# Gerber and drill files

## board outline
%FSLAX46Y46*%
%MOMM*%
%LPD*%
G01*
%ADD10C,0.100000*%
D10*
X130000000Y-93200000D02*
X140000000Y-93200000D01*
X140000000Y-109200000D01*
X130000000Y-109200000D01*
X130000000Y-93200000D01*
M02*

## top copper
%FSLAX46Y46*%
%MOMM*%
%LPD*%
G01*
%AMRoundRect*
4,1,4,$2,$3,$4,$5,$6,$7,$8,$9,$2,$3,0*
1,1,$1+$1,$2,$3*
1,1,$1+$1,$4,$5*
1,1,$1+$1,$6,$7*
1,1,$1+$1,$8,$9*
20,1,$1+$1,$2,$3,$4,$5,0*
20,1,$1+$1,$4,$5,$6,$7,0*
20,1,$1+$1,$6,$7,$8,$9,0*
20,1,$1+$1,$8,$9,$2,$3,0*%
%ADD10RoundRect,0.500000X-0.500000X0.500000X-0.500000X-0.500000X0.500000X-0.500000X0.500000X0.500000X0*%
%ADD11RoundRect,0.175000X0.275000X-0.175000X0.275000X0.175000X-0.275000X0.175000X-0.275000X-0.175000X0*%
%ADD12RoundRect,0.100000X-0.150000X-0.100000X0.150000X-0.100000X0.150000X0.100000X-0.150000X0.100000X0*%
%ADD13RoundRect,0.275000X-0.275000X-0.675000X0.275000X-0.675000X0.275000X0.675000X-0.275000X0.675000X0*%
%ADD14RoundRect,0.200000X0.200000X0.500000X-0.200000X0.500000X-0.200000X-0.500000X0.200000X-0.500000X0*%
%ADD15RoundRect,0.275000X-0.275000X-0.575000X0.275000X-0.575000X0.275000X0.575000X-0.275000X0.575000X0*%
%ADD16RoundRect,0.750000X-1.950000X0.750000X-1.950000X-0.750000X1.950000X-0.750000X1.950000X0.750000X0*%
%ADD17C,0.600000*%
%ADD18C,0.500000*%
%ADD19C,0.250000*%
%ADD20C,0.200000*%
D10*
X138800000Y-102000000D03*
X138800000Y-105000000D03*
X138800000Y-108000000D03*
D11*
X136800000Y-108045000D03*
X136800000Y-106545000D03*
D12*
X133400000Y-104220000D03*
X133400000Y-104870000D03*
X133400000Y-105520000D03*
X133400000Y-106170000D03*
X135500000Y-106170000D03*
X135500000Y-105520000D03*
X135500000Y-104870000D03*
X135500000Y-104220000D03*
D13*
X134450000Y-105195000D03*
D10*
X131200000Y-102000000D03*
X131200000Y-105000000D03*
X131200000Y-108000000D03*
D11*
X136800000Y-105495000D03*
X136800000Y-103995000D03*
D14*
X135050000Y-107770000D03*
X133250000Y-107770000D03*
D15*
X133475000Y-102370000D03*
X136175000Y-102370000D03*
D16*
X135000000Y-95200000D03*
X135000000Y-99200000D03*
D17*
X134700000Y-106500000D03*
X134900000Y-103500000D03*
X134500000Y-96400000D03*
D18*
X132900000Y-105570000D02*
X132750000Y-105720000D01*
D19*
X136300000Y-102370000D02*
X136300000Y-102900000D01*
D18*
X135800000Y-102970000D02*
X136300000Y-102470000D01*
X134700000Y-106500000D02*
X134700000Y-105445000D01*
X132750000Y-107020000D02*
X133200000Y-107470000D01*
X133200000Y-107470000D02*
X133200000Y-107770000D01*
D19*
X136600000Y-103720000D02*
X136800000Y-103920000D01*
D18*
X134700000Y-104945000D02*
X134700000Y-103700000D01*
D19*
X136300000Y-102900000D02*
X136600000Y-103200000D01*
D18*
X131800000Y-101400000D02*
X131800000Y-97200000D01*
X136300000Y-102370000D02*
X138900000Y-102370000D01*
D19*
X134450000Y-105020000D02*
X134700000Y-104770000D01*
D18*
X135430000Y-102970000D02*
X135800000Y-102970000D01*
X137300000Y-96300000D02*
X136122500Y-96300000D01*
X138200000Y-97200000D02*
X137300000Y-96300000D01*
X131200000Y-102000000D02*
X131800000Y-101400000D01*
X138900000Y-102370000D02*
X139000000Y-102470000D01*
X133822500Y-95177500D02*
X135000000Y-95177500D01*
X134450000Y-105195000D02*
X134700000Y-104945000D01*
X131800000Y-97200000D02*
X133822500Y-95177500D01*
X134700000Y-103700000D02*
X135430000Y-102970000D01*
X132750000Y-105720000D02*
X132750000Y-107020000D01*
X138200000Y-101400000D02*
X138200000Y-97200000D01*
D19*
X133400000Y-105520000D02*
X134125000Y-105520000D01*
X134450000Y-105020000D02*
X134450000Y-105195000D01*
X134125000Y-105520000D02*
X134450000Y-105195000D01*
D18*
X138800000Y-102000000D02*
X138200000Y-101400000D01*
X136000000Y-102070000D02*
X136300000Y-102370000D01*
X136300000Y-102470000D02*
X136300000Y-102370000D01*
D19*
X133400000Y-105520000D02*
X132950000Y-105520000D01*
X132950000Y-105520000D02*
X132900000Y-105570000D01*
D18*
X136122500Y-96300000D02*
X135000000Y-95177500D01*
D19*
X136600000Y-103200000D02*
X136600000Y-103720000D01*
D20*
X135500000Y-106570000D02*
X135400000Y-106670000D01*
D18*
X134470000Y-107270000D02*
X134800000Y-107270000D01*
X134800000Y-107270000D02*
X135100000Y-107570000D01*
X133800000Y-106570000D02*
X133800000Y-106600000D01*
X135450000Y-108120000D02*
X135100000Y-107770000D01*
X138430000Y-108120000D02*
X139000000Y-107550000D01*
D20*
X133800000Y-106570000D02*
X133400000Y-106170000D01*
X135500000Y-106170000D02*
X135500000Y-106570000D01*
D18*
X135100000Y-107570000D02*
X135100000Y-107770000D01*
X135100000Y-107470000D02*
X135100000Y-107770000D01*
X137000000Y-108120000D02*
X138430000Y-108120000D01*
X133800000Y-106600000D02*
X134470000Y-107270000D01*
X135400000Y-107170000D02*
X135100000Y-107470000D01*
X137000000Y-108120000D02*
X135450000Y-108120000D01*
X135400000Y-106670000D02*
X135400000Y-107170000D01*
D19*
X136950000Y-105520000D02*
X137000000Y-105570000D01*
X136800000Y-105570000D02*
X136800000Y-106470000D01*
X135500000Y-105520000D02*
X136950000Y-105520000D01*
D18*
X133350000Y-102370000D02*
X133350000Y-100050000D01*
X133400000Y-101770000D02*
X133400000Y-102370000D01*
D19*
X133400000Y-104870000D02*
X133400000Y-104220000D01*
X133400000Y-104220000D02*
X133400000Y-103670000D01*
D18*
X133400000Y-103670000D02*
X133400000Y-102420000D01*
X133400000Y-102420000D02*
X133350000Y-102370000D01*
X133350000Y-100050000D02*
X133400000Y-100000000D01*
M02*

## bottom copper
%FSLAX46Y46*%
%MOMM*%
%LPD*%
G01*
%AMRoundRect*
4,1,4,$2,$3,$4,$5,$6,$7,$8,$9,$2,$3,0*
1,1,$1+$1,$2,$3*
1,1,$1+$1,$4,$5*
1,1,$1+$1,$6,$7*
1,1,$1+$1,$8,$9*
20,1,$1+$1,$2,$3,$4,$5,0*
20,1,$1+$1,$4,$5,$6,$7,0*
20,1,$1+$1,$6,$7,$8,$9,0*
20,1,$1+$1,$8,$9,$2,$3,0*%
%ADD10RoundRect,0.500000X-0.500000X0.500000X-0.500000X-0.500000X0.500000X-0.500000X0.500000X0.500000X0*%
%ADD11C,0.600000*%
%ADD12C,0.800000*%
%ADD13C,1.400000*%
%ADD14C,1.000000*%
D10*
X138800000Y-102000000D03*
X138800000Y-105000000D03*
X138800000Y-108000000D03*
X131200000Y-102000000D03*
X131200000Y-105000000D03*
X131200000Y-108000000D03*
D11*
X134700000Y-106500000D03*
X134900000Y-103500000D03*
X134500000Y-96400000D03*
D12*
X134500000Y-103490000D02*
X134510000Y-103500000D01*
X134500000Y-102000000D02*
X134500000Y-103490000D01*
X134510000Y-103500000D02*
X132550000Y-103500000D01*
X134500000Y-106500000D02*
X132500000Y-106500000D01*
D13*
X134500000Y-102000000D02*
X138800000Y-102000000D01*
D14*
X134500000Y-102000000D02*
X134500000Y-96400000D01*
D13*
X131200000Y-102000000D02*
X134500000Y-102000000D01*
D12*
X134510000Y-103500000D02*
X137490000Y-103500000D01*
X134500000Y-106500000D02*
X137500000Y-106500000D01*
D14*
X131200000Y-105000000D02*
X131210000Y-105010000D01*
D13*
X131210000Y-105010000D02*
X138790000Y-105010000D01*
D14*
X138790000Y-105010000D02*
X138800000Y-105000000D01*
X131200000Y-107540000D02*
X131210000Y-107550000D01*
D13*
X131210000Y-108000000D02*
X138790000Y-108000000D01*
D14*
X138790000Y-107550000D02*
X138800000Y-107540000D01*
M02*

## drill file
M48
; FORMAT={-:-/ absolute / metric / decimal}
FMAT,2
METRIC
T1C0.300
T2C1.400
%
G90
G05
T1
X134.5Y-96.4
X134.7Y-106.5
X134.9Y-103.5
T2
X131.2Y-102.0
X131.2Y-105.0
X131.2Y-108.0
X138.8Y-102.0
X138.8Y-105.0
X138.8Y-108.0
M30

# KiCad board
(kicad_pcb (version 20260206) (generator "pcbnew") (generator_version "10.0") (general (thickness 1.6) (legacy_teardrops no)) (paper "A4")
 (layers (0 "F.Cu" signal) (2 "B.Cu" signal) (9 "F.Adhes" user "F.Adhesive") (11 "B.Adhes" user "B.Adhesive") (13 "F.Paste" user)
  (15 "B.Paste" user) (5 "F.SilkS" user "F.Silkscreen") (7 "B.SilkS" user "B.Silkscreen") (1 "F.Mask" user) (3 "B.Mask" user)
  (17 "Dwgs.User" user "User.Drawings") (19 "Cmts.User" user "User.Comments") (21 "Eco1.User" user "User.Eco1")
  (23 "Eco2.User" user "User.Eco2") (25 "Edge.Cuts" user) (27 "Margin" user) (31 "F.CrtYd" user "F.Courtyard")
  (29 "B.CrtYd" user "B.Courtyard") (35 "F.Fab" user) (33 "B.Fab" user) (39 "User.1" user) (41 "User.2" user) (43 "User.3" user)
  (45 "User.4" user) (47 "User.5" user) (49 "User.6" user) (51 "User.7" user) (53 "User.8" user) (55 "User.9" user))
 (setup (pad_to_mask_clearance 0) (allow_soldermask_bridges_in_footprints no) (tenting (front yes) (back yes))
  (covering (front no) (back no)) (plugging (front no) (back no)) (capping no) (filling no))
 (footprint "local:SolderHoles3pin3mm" (layer "F.Cu") (at 138.8 105 -90)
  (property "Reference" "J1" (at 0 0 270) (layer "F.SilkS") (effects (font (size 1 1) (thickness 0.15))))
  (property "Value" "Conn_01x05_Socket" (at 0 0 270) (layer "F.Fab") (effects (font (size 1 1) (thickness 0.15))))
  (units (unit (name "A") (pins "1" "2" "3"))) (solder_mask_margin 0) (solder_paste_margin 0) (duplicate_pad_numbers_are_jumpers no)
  (pad "1" thru_hole roundrect (at -3 0 270) (size 2 2) (drill 1.4) (layers "*.Cu" "*.Mask") (remove_unused_layers yes)
   (keep_end_layers yes) (zone_layer_connections) (roundrect_rratio 0.25) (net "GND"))
  (pad "2" thru_hole roundrect (at 0 0 270) (size 2 2) (drill 1.4) (layers "*.Cu" "*.Mask") (remove_unused_layers yes) (keep_end_layers yes)
   (zone_layer_connections) (roundrect_rratio 0.25) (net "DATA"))
  (pad "3" thru_hole roundrect (at 3 0 270) (size 2 2) (drill 1.4) (layers "*.Cu" "*.Mask") (remove_unused_layers yes) (keep_end_layers yes)
   (zone_layer_connections) (roundrect_rratio 0.25) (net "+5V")))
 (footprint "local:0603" (layer "F.Cu") (at 136.8 107.295 90)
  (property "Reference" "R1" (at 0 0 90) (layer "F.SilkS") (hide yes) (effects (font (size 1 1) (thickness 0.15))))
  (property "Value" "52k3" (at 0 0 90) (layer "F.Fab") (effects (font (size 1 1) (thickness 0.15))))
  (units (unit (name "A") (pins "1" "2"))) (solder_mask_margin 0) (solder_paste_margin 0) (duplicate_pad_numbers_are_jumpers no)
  (pad "1" smd roundrect (at -0.75 0 90) (size 0.7 0.9) (layers "F.Cu" "F.Mask" "F.Paste") (roundrect_rratio 0.25) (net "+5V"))
  (pad "2" smd roundrect (at 0.75 0 90) (size 0.7 0.9) (layers "F.Cu" "F.Mask" "F.Paste") (roundrect_rratio 0.25) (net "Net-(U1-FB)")))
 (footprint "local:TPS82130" (layer "F.Cu") (at 134.45 105.195)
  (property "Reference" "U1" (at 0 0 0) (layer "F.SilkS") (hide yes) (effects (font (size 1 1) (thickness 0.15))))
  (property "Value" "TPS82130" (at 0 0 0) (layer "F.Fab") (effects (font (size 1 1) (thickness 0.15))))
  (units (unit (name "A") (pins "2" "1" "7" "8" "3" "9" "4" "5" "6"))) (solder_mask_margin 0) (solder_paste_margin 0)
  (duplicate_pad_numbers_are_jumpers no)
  (pad "1" smd roundrect (at -1.05 -0.975) (size 0.5 0.4) (layers "F.Cu" "F.Mask" "F.Paste") (roundrect_rratio 0.25) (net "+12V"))
  (pad "2" smd roundrect (at -1.05 -0.325) (size 0.5 0.4) (layers "F.Cu" "F.Mask" "F.Paste") (roundrect_rratio 0.25) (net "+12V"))
  (pad "3" smd roundrect (at -1.05 0.325) (size 0.5 0.4) (layers "F.Cu" "F.Mask" "F.Paste") (roundrect_rratio 0.25) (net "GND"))
  (pad "4" smd roundrect (at -1.05 0.975) (size 0.5 0.4) (layers "F.Cu" "F.Mask" "F.Paste") (roundrect_rratio 0.25) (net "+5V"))
  (pad "5" smd roundrect (at 1.05 0.975) (size 0.5 0.4) (layers "F.Cu" "F.Mask" "F.Paste") (roundrect_rratio 0.25) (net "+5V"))
  (pad "6" smd roundrect (at 1.05 0.325) (size 0.5 0.4) (layers "F.Cu" "F.Mask" "F.Paste") (roundrect_rratio 0.25) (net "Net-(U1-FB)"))
  (pad "7" smd roundrect (at 1.05 -0.325) (size 0.5 0.4) (layers "F.Cu" "F.Mask" "F.Paste") (roundrect_rratio 0.25)
   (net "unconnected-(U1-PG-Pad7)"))
  (pad "8" smd roundrect (at 1.05 -0.975) (size 0.5 0.4) (layers "F.Cu" "F.Mask" "F.Paste") (roundrect_rratio 0.25)
   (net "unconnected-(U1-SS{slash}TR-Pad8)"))
  (pad "9" smd roundrect (at 0 0) (size 1.1 1.9) (layers "F.Cu" "F.Mask" "F.Paste") (roundrect_rratio 0.25) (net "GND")))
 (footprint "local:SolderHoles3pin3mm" (layer "F.Cu") (at 131.2 105 -90)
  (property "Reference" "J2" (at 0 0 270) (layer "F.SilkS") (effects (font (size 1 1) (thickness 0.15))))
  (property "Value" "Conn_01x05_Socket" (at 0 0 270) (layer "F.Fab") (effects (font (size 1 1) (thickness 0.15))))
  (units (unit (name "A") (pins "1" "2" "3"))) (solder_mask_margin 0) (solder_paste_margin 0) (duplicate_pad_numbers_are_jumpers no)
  (pad "1" thru_hole roundrect (at -3 0 270) (size 2 2) (drill 1.4) (layers "*.Cu" "*.Mask") (remove_unused_layers yes)
   (keep_end_layers yes) (zone_layer_connections) (roundrect_rratio 0.25) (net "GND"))
  (pad "2" thru_hole roundrect (at 0 0 270) (size 2 2) (drill 1.4) (layers "*.Cu" "*.Mask") (remove_unused_layers yes) (keep_end_layers yes)
   (zone_layer_connections) (roundrect_rratio 0.25) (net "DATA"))
  (pad "3" thru_hole roundrect (at 3 0 270) (size 2 2) (drill 1.4) (layers "*.Cu" "*.Mask") (remove_unused_layers yes) (keep_end_layers yes)
   (zone_layer_connections) (roundrect_rratio 0.25) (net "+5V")))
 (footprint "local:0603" (layer "F.Cu") (at 136.8 104.745 90)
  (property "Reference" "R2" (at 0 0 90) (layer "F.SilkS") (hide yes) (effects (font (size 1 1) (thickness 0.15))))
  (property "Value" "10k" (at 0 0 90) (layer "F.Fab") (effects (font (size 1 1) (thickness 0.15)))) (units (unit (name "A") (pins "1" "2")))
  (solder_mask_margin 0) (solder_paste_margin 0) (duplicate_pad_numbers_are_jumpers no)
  (pad "1" smd roundrect (at -0.75 0 90) (size 0.7 0.9) (layers "F.Cu" "F.Mask" "F.Paste") (roundrect_rratio 0.25) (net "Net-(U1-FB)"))
  (pad "2" smd roundrect (at 0.75 0 90) (size 0.7 0.9) (layers "F.Cu" "F.Mask" "F.Paste") (roundrect_rratio 0.25) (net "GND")))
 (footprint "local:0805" (layer "F.Cu") (at 134.15 107.77 180)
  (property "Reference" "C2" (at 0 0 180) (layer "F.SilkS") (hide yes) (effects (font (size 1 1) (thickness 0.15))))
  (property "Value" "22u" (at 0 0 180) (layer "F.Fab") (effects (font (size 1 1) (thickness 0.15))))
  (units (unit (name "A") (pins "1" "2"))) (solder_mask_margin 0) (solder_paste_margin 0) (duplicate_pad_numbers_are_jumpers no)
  (pad "1" smd roundrect (at -0.9 0 180) (size 0.8 1.4) (layers "F.Cu" "F.Mask" "F.Paste") (roundrect_rratio 0.25) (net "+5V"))
  (pad "2" smd roundrect (at 0.9 0 180) (size 0.8 1.4) (layers "F.Cu" "F.Mask" "F.Paste") (roundrect_rratio 0.25) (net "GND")))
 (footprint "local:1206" (layer "F.Cu") (at 134.825 102.37)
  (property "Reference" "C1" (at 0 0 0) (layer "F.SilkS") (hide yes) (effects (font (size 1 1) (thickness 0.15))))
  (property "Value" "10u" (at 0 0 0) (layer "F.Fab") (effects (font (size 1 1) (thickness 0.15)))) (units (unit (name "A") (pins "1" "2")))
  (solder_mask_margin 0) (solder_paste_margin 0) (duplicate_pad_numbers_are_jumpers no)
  (pad "1" smd roundrect (at -1.35 0) (size 1.1 1.7) (layers "F.Cu" "F.Mask" "F.Paste") (roundrect_rratio 0.25) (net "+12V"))
  (pad "2" smd roundrect (at 1.35 0) (size 1.1 1.7) (layers "F.Cu" "F.Mask" "F.Paste") (roundrect_rratio 0.25) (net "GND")))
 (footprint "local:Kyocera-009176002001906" (layer "F.Cu") (at 135 97.2 -90)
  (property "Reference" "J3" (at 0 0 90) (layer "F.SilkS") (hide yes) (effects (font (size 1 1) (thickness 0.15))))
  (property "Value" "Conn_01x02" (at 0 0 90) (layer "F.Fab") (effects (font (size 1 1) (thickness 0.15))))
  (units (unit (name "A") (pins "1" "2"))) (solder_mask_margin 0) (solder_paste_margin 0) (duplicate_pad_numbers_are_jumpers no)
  (pad "1" smd roundrect (at -2 0 270) (size 3 5.4) (layers "F.Cu" "F.Mask" "F.Paste") (roundrect_rratio 0.25) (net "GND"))
  (pad "2" smd roundrect (at 2 0 270) (size 3 5.4) (layers "F.Cu" "F.Mask" "F.Paste") (roundrect_rratio 0.25) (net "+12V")))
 (gr_rect (start 130 93.2) (end 140 109.2) (stroke (width 0.1) (type default)) (fill no) (layer "Edge.Cuts"))
 (segment (start 132.9 105.57) (end 132.75 105.72) (width 0.5) (layer "F.Cu") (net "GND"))
 (segment (start 136.3 102.37) (end 136.3 102.9) (width 0.25) (layer "F.Cu") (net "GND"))
 (segment (start 135.8 102.97) (end 136.3 102.47) (width 0.5) (layer "F.Cu") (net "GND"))
 (segment (start 134.7 106.5) (end 134.7 105.445) (width 0.5) (layer "F.Cu") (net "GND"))
 (segment (start 132.75 107.02) (end 133.2 107.47) (width 0.5) (layer "F.Cu") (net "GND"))
 (segment (start 133.2 107.47) (end 133.2 107.77) (width 0.5) (layer "F.Cu") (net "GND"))
 (segment (start 136.6 103.72) (end 136.8 103.92) (width 0.25) (layer "F.Cu") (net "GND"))
 (segment (start 134.7 104.945) (end 134.7 103.7) (width 0.5) (layer "F.Cu") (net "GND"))
 (segment (start 136.3 102.9) (end 136.6 103.2) (width 0.25) (layer "F.Cu") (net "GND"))
 (segment (start 131.8 101.4) (end 131.8 97.2) (width 0.5) (layer "F.Cu") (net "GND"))
 (segment (start 136.3 102.37) (end 138.9 102.37) (width 0.5) (layer "F.Cu") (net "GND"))
 (segment (start 134.45 105.02) (end 134.7 104.77) (width 0.25) (layer "F.Cu") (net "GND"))
 (segment (start 135.43 102.97) (end 135.8 102.97) (width 0.5) (layer "F.Cu") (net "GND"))
 (segment (start 137.3 96.3) (end 136.1225 96.3) (width 0.5) (layer "F.Cu") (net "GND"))
 (segment (start 138.2 97.2) (end 137.3 96.3) (width 0.5) (layer "F.Cu") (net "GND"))
 (segment (start 131.2 102) (end 131.8 101.4) (width 0.5) (layer "F.Cu") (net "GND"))
 (segment (start 138.9 102.37) (end 139 102.47) (width 0.5) (layer "F.Cu") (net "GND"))
 (segment (start 133.8225 95.1775) (end 135 95.1775) (width 0.5) (layer "F.Cu") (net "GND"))
 (segment (start 134.45 105.195) (end 134.7 104.945) (width 0.5) (layer "F.Cu") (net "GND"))
 (segment (start 131.8 97.2) (end 133.8225 95.1775) (width 0.5) (layer "F.Cu") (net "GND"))
 (segment (start 134.7 103.7) (end 135.43 102.97) (width 0.5) (layer "F.Cu") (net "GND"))
 (segment (start 132.75 105.72) (end 132.75 107.02) (width 0.5) (layer "F.Cu") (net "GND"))
 (segment (start 138.2 101.4) (end 138.2 97.2) (width 0.5) (layer "F.Cu") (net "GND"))
 (segment (start 133.4 105.52) (end 134.125 105.52) (width 0.25) (layer "F.Cu") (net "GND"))
 (segment (start 134.45 105.02) (end 134.45 105.195) (width 0.25) (layer "F.Cu") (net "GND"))
 (segment (start 134.125 105.52) (end 134.45 105.195) (width 0.25) (layer "F.Cu") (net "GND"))
 (segment (start 138.8 102) (end 138.2 101.4) (width 0.5) (layer "F.Cu") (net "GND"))
 (segment (start 136 102.07) (end 136.3 102.37) (width 0.5) (layer "F.Cu") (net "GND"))
 (segment (start 136.3 102.47) (end 136.3 102.37) (width 0.5) (layer "F.Cu") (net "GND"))
 (segment (start 133.4 105.52) (end 132.95 105.52) (width 0.25) (layer "F.Cu") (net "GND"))
 (segment (start 132.95 105.52) (end 132.9 105.57) (width 0.25) (layer "F.Cu") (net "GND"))
 (segment (start 136.1225 96.3) (end 135 95.1775) (width 0.5) (layer "F.Cu") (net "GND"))
 (segment (start 136.6 103.2) (end 136.6 103.72) (width 0.25) (layer "F.Cu") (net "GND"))
 (via (at 134.7 106.5) (size 0.6) (drill 0.3) (layers "F.Cu" "B.Cu") (capping no) (covering (front no) (back no))
  (plugging (front no) (back no)) (filling no) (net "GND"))
 (via (at 134.9 103.5) (size 0.6) (drill 0.3) (layers "F.Cu" "B.Cu") (capping no) (covering (front no) (back no))
  (plugging (front no) (back no)) (filling no) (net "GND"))
 (via (at 134.5 96.4) (size 0.6) (drill 0.3) (layers "F.Cu" "B.Cu") (capping no) (covering (front no) (back no))
  (plugging (front no) (back no)) (filling no) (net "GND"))
 (segment (start 134.5 103.49) (end 134.51 103.5) (width 0.8) (layer "B.Cu") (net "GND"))
 (segment (start 134.5 102) (end 134.5 103.49) (width 0.8) (layer "B.Cu") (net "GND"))
 (segment (start 134.51 103.5) (end 132.55 103.5) (width 0.8) (layer "B.Cu") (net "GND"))
 (segment (start 134.5 106.5) (end 132.5 106.5) (width 0.8) (layer "B.Cu") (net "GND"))
 (segment (start 134.5 102) (end 138.8 102) (width 1.4) (layer "B.Cu") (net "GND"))
 (segment (start 134.5 102) (end 134.5 96.4) (width 1) (layer "B.Cu") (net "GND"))
 (segment (start 131.2 102) (end 134.5 102) (width 1.4) (layer "B.Cu") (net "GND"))
 (segment (start 134.51 103.5) (end 137.49 103.5) (width 0.8) (layer "B.Cu") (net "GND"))
 (segment (start 134.5 106.5) (end 137.5 106.5) (width 0.8) (layer "B.Cu") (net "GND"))
 (segment (start 131.2 105) (end 131.21 105.01) (width 1) (layer "B.Cu") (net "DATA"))
 (segment (start 131.21 105.01) (end 138.79 105.01) (width 1.4) (layer "B.Cu") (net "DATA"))
 (segment (start 138.79 105.01) (end 138.8 105) (width 1) (layer "B.Cu") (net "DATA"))
 (segment (start 135.5 106.57) (end 135.4 106.67) (width 0.2) (layer "F.Cu") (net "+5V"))
 (segment (start 134.47 107.27) (end 134.8 107.27) (width 0.5) (layer "F.Cu") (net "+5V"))
 (segment (start 134.8 107.27) (end 135.1 107.57) (width 0.5) (layer "F.Cu") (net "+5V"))
 (segment (start 133.8 106.57) (end 133.8 106.6) (width 0.5) (layer "F.Cu") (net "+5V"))
 (segment (start 135.45 108.12) (end 135.1 107.77) (width 0.5) (layer "F.Cu") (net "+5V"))
 (segment (start 138.43 108.12) (end 139 107.55) (width 0.5) (layer "F.Cu") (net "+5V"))
 (segment (start 133.8 106.57) (end 133.4 106.17) (width 0.2) (layer "F.Cu") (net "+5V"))
 (segment (start 135.5 106.17) (end 135.5 106.57) (width 0.2) (layer "F.Cu") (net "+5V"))
 (segment (start 135.1 107.57) (end 135.1 107.77) (width 0.5) (layer "F.Cu") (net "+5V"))
 (segment (start 135.1 107.47) (end 135.1 107.77) (width 0.5) (layer "F.Cu") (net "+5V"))
 (segment (start 137 108.12) (end 138.43 108.12) (width 0.5) (layer "F.Cu") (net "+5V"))
 (segment (start 133.8 106.6) (end 134.47 107.27) (width 0.5) (layer "F.Cu") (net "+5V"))
 (segment (start 135.4 107.17) (end 135.1 107.47) (width 0.5) (layer "F.Cu") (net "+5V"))
 (segment (start 137 108.12) (end 135.45 108.12) (width 0.5) (layer "F.Cu") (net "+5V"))
 (segment (start 135.4 106.67) (end 135.4 107.17) (width 0.5) (layer "F.Cu") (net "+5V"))
 (segment (start 131.2 107.54) (end 131.21 107.55) (width 1) (layer "B.Cu") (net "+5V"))
 (segment (start 131.21 108) (end 138.79 108) (width 1.4) (layer "B.Cu") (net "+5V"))
 (segment (start 138.79 107.55) (end 138.8 107.54) (width 1) (layer "B.Cu") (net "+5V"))
 (segment (start 136.95 105.52) (end 137 105.57) (width 0.25) (layer "F.Cu") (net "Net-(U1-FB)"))
 (segment (start 136.8 105.57) (end 136.8 106.47) (width 0.25) (layer "F.Cu") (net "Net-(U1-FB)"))
 (segment (start 135.5 105.52) (end 136.95 105.52) (width 0.25) (layer "F.Cu") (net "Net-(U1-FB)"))
 (segment (start 133.35 102.37) (end 133.35 100.05) (width 0.5) (layer "F.Cu") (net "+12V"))
 (segment (start 133.4 101.77) (end 133.4 102.37) (width 0.5) (layer "F.Cu") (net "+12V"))
 (segment (start 133.4 104.87) (end 133.4 104.22) (width 0.25) (layer "F.Cu") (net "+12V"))
 (segment (start 133.4 104.22) (end 133.4 103.67) (width 0.25) (layer "F.Cu") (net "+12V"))
 (segment (start 133.4 103.67) (end 133.4 102.42) (width 0.5) (layer "F.Cu") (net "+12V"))
 (segment (start 133.4 102.42) (end 133.35 102.37) (width 0.5) (layer "F.Cu") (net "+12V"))
 (segment (start 133.35 100.05) (end 133.4 100) (width 0.5) (layer "F.Cu") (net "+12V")))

